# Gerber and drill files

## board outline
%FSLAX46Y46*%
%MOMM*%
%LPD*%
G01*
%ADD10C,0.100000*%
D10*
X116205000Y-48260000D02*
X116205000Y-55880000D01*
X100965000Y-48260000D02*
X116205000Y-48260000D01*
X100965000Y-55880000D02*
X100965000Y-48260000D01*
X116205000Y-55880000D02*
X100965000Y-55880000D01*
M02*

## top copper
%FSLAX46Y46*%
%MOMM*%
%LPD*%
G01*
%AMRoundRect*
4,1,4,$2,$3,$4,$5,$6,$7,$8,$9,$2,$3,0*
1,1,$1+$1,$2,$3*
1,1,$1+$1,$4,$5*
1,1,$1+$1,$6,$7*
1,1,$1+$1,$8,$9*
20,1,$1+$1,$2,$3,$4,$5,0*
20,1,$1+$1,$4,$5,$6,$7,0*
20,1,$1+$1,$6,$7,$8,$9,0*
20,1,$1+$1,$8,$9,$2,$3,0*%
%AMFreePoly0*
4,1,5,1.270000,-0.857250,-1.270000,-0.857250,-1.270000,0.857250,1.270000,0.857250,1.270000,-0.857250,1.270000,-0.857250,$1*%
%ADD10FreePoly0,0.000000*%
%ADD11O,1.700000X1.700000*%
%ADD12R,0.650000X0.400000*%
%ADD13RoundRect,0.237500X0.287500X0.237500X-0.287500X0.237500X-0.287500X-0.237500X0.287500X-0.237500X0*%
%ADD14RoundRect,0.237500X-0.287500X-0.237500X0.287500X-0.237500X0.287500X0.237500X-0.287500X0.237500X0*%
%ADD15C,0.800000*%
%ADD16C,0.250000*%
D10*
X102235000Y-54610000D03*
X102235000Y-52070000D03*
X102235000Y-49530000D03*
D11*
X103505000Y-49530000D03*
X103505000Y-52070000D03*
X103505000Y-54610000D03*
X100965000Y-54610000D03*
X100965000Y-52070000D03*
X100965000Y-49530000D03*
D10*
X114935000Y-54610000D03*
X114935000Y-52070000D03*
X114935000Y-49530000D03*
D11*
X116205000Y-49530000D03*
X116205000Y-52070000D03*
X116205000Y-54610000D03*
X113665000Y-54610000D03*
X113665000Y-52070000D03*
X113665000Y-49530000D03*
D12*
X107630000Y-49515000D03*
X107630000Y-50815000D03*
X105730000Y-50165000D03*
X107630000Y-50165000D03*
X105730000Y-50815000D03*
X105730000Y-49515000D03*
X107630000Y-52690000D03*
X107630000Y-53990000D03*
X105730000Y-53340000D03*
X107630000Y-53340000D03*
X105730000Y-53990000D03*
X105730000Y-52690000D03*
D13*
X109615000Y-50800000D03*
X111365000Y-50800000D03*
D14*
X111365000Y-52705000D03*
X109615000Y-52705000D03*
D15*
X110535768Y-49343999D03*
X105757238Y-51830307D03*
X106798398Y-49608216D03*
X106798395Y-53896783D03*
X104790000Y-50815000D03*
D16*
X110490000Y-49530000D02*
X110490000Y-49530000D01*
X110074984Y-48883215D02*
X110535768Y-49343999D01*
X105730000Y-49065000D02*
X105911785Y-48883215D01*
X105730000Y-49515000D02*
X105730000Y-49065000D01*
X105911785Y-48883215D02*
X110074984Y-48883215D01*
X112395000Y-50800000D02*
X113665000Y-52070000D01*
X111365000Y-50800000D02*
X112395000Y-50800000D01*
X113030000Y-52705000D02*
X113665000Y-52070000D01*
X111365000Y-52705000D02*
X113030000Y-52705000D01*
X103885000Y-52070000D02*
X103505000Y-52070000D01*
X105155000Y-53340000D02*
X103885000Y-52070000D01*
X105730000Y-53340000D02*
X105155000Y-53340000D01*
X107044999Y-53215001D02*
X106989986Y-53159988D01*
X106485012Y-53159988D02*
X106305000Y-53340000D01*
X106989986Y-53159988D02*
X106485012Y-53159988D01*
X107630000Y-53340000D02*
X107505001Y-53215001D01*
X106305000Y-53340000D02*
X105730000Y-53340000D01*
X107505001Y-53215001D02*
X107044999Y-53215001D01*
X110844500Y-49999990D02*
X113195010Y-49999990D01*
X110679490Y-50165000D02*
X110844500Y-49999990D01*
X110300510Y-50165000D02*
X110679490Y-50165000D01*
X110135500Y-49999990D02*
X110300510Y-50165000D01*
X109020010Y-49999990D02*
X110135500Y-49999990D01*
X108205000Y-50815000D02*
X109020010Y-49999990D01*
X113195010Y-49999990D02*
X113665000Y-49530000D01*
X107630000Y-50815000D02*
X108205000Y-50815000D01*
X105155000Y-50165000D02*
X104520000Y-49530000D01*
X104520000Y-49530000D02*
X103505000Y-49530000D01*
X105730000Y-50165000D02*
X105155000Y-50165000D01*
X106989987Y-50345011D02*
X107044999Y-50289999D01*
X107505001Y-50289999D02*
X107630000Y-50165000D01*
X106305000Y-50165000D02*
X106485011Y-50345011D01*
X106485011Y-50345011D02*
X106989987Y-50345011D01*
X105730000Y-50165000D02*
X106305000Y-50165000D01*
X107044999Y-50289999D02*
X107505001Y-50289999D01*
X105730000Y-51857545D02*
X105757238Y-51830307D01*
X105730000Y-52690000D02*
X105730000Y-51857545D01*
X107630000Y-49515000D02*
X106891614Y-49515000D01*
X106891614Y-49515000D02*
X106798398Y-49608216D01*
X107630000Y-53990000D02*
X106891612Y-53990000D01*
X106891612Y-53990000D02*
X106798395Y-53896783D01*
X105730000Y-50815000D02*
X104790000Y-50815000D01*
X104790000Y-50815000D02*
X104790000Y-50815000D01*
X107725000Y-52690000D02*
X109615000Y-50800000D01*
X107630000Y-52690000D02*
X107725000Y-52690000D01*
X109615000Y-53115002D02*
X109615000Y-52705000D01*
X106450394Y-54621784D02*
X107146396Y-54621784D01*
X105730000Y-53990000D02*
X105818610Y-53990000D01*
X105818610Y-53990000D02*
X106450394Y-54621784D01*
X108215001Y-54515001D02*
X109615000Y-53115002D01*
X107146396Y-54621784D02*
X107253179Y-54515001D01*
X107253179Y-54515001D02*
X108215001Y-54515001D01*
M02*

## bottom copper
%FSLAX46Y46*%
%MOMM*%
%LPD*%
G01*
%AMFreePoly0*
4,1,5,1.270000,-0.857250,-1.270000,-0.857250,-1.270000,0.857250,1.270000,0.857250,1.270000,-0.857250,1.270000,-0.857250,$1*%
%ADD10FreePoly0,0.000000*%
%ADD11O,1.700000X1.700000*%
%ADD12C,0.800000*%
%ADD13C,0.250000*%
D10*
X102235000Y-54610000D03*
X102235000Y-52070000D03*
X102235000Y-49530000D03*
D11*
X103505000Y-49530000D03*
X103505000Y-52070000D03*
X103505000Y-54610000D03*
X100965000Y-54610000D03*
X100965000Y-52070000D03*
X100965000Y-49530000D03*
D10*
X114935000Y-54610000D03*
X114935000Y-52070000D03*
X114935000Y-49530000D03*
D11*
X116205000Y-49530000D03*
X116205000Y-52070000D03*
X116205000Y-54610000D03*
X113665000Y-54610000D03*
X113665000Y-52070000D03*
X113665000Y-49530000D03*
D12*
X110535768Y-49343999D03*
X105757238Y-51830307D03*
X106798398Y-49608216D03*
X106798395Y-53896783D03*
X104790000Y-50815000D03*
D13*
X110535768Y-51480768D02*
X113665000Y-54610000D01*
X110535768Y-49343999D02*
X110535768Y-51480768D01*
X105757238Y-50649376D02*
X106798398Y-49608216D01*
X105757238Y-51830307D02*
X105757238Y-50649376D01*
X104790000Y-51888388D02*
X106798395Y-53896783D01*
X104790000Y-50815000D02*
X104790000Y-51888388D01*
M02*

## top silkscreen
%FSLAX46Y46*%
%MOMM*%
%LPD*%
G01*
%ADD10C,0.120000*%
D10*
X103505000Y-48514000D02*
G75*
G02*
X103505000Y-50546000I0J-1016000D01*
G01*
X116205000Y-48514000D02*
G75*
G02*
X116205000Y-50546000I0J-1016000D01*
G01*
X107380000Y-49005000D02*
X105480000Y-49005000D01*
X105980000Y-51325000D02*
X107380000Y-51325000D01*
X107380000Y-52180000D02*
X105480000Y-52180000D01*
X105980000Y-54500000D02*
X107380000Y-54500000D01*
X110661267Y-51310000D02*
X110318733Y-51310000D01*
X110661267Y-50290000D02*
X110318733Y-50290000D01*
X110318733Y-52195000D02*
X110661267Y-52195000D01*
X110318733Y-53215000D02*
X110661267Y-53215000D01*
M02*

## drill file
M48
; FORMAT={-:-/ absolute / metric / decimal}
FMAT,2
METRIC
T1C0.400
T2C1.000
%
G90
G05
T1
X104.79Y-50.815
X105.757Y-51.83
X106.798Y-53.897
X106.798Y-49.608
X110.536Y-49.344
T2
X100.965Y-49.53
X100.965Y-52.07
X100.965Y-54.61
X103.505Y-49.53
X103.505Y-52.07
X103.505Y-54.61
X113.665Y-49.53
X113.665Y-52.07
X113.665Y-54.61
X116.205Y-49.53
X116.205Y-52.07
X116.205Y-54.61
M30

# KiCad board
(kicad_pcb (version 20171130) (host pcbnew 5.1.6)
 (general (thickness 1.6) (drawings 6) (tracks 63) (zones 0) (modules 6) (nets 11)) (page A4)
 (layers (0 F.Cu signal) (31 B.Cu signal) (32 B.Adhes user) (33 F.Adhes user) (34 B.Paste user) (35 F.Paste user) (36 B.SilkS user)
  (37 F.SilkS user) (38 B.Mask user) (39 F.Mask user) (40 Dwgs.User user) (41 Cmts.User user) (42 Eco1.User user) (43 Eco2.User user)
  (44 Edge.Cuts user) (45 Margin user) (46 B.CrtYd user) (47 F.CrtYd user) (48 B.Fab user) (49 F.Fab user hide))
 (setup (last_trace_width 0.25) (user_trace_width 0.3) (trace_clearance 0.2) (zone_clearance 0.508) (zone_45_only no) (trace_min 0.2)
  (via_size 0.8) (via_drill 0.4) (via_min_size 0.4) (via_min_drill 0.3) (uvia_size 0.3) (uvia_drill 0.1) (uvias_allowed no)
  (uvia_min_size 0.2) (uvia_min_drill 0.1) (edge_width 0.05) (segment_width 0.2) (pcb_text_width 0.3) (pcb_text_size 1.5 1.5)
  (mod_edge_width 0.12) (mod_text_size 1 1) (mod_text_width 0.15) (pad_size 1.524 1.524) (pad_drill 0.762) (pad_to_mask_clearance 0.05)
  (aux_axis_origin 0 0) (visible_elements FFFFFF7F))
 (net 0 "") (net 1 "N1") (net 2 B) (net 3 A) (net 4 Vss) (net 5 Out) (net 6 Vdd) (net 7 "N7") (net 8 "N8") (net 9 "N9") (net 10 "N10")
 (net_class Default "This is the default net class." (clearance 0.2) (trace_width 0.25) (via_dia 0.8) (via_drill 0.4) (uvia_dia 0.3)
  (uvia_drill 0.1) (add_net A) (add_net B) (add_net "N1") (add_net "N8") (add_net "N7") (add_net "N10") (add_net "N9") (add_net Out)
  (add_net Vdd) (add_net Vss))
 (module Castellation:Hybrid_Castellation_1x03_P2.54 (layer F.Cu) (at 102.235 49.53)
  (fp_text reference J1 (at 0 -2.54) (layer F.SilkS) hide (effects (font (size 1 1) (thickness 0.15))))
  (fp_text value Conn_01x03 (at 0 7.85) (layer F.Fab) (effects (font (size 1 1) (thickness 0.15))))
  (fp_arc (start 1.27 0) (end 1.27 1.016) (angle -180) (layer F.SilkS) (width 0.12))
  (pad 3 connect custom (at 0 5.08) (size 2.54 1.7145) (layers B.Cu B.Mask) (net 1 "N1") (zone_connect 0)
   (options (clearance outline) (anchor rect)) (primitives))
  (pad 2 connect custom (at 0 2.54) (size 2.54 1.7145) (layers B.Cu B.Mask) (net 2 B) (zone_connect 0)
   (options (clearance outline) (anchor rect)) (primitives))
  (pad 1 connect custom (at 0 0) (size 2.54 1.7145) (layers B.Cu B.Mask) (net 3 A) (zone_connect 0)
   (options (clearance outline) (anchor rect)) (primitives))
  (pad 3 connect custom (at 0 5.08) (size 2.54 1.7145) (layers F.Cu F.Mask) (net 1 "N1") (zone_connect 0)
   (options (clearance outline) (anchor rect)) (primitives))
  (pad 2 connect custom (at 0 2.54) (size 2.54 1.7145) (layers F.Cu F.Mask) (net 2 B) (zone_connect 0)
   (options (clearance outline) (anchor rect)) (primitives))
  (pad 1 connect custom (at 0 0) (size 2.54 1.7145) (layers F.Cu F.Mask) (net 3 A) (zone_connect 0)
   (options (clearance outline) (anchor rect)) (primitives))
  (pad 1 thru_hole oval (at 1.27 0) (size 1.7 1.7) (drill 1) (layers *.Cu *.Mask) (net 3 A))
  (pad 2 thru_hole oval (at 1.27 2.54) (size 1.7 1.7) (drill 1) (layers *.Cu *.Mask) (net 2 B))
  (pad 3 thru_hole oval (at 1.27 5.08) (size 1.7 1.7) (drill 1) (layers *.Cu *.Mask) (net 1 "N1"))
  (pad 3 thru_hole oval (at -1.27 5.08) (size 1.7 1.7) (drill 1) (layers *.Cu *.Mask) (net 1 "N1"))
  (pad 2 thru_hole oval (at -1.27 2.54) (size 1.7 1.7) (drill 1) (layers *.Cu *.Mask) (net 2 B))
  (pad 1 thru_hole oval (at -1.27 0) (size 1.7 1.7) (drill 1) (layers *.Cu *.Mask) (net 3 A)))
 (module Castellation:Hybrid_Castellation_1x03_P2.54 (layer F.Cu) (at 114.935 49.53)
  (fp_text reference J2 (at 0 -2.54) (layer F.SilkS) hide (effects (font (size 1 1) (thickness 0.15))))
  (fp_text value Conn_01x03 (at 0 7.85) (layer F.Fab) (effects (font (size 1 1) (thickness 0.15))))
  (fp_arc (start 1.27 0) (end 1.27 1.016) (angle -180) (layer F.SilkS) (width 0.12))
  (pad 3 connect custom (at 0 5.08) (size 2.54 1.7145) (layers B.Cu B.Mask) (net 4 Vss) (zone_connect 0)
   (options (clearance outline) (anchor rect)) (primitives))
  (pad 2 connect custom (at 0 2.54) (size 2.54 1.7145) (layers B.Cu B.Mask) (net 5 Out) (zone_connect 0)
   (options (clearance outline) (anchor rect)) (primitives))
  (pad 1 connect custom (at 0 0) (size 2.54 1.7145) (layers B.Cu B.Mask) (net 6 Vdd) (zone_connect 0)
   (options (clearance outline) (anchor rect)) (primitives))
  (pad 3 connect custom (at 0 5.08) (size 2.54 1.7145) (layers F.Cu F.Mask) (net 4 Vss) (zone_connect 0)
   (options (clearance outline) (anchor rect)) (primitives))
  (pad 2 connect custom (at 0 2.54) (size 2.54 1.7145) (layers F.Cu F.Mask) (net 5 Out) (zone_connect 0)
   (options (clearance outline) (anchor rect)) (primitives))
  (pad 1 connect custom (at 0 0) (size 2.54 1.7145) (layers F.Cu F.Mask) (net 6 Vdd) (zone_connect 0)
   (options (clearance outline) (anchor rect)) (primitives))
  (pad 1 thru_hole oval (at 1.27 0) (size 1.7 1.7) (drill 1) (layers *.Cu *.Mask) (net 6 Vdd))
  (pad 2 thru_hole oval (at 1.27 2.54) (size 1.7 1.7) (drill 1) (layers *.Cu *.Mask) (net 5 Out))
  (pad 3 thru_hole oval (at 1.27 5.08) (size 1.7 1.7) (drill 1) (layers *.Cu *.Mask) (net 4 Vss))
  (pad 3 thru_hole oval (at -1.27 5.08) (size 1.7 1.7) (drill 1) (layers *.Cu *.Mask) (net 4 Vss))
  (pad 2 thru_hole oval (at -1.27 2.54) (size 1.7 1.7) (drill 1) (layers *.Cu *.Mask) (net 5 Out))
  (pad 1 thru_hole oval (at -1.27 0) (size 1.7 1.7) (drill 1) (layers *.Cu *.Mask) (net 6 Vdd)))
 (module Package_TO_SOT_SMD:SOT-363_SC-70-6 (layer F.Cu) (at 106.68 50.165)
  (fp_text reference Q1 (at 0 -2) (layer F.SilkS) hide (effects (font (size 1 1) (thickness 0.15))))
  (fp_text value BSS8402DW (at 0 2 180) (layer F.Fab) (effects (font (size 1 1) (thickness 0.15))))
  (fp_line (start 0.7 -1.16) (end -1.2 -1.16) (layer F.SilkS) (width 0.12))
  (fp_line (start -0.7 1.16) (end 0.7 1.16) (layer F.SilkS) (width 0.12))
  (pad 6 smd rect (at 0.95 -0.65) (size 0.65 0.4) (layers F.Cu F.Paste F.Mask) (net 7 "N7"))
  (pad 4 smd rect (at 0.95 0.65) (size 0.65 0.4) (layers F.Cu F.Paste F.Mask) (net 6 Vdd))
  (pad 2 smd rect (at -0.95 0) (size 0.65 0.4) (layers F.Cu F.Paste F.Mask) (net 3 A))
  (pad 5 smd rect (at 0.95 0) (size 0.65 0.4) (layers F.Cu F.Paste F.Mask) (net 3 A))
  (pad 3 smd rect (at -0.95 0.65) (size 0.65 0.4) (layers F.Cu F.Paste F.Mask) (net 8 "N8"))
  (pad 1 smd rect (at -0.95 -0.65) (size 0.65 0.4) (layers F.Cu F.Paste F.Mask) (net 4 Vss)))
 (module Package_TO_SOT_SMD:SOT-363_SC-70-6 (layer F.Cu) (at 106.68 53.34)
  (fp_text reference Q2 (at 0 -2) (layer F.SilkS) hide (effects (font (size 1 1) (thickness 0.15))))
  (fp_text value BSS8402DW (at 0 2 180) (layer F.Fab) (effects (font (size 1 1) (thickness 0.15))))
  (fp_line (start 0.7 -1.16) (end -1.2 -1.16) (layer F.SilkS) (width 0.12))
  (fp_line (start -0.7 1.16) (end 0.7 1.16) (layer F.SilkS) (width 0.12))
  (pad 6 smd rect (at 0.95 -0.65) (size 0.65 0.4) (layers F.Cu F.Paste F.Mask) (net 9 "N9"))
  (pad 4 smd rect (at 0.95 0.65) (size 0.65 0.4) (layers F.Cu F.Paste F.Mask) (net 8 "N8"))
  (pad 2 smd rect (at -0.95 0) (size 0.65 0.4) (layers F.Cu F.Paste F.Mask) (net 2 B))
  (pad 5 smd rect (at 0.95 0) (size 0.65 0.4) (layers F.Cu F.Paste F.Mask) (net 2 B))
  (pad 3 smd rect (at -0.95 0.65) (size 0.65 0.4) (layers F.Cu F.Paste F.Mask) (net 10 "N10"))
  (pad 1 smd rect (at -0.95 -0.65) (size 0.65 0.4) (layers F.Cu F.Paste F.Mask) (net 7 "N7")))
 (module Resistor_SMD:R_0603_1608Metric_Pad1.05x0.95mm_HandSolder (layer F.Cu) (at 110.49 50.8 180)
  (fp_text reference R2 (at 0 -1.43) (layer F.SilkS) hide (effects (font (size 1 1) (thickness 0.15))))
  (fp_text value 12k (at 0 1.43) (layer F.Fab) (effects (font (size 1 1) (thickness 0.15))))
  (fp_line (start -0.171267 -0.51) (end 0.171267 -0.51) (layer F.SilkS) (width 0.12))
  (fp_line (start -0.171267 0.51) (end 0.171267 0.51) (layer F.SilkS) (width 0.12))
  (pad 2 smd roundrect (at 0.875 0 180) (size 1.05 0.95) (layers F.Cu F.Paste F.Mask) (roundrect_rratio 0.25) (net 9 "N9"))
  (pad 1 smd roundrect (at -0.875 0 180) (size 1.05 0.95) (layers F.Cu F.Paste F.Mask) (roundrect_rratio 0.25) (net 5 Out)))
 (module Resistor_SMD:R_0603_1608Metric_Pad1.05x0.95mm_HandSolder (layer F.Cu) (at 110.49 52.705)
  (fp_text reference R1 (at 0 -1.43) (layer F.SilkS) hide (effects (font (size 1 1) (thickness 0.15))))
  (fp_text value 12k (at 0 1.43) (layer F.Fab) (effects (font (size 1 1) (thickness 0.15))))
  (fp_line (start -0.171267 -0.51) (end 0.171267 -0.51) (layer F.SilkS) (width 0.12))
  (fp_line (start -0.171267 0.51) (end 0.171267 0.51) (layer F.SilkS) (width 0.12))
  (pad 2 smd roundrect (at 0.875 0) (size 1.05 0.95) (layers F.Cu F.Paste F.Mask) (roundrect_rratio 0.25) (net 5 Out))
  (pad 1 smd roundrect (at -0.875 0) (size 1.05 0.95) (layers F.Cu F.Paste F.Mask) (roundrect_rratio 0.25) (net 10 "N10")))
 (gr_line (start 116.205 48.26) (end 116.205 55.88) (layer Edge.Cuts) (width 0.1))
 (gr_line (start 100.965 48.26) (end 116.205 48.26) (layer Edge.Cuts) (width 0.1))
 (gr_line (start 100.965 55.88) (end 100.965 48.26) (layer Edge.Cuts) (width 0.1))
 (gr_line (start 116.205 55.88) (end 100.965 55.88) (layer Edge.Cuts) (width 0.1))
 (segment (start 110.49 49.53) (end 110.49 49.53) (width 0.25) (layer F.Cu) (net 4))
 (via (at 110.535768 49.343999) (size 0.8) (drill 0.4) (layers F.Cu B.Cu) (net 4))
 (segment (start 110.074984 48.883215) (end 110.535768 49.343999) (width 0.25) (layer F.Cu) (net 4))
 (segment (start 105.73 49.065) (end 105.911785 48.883215) (width 0.25) (layer F.Cu) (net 4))
 (segment (start 105.73 49.515) (end 105.73 49.065) (width 0.25) (layer F.Cu) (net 4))
 (segment (start 105.911785 48.883215) (end 110.074984 48.883215) (width 0.25) (layer F.Cu) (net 4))
 (segment (start 110.535768 51.480768) (end 113.665 54.61) (width 0.25) (layer B.Cu) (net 4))
 (segment (start 110.535768 49.343999) (end 110.535768 51.480768) (width 0.25) (layer B.Cu) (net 4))
 (segment (start 112.395 50.8) (end 113.665 52.07) (width 0.25) (layer F.Cu) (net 5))
 (segment (start 111.365 50.8) (end 112.395 50.8) (width 0.25) (layer F.Cu) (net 5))
 (segment (start 113.03 52.705) (end 113.665 52.07) (width 0.25) (layer F.Cu) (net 5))
 (segment (start 111.365 52.705) (end 113.03 52.705) (width 0.25) (layer F.Cu) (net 5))
 (segment (start 103.885 52.07) (end 103.505 52.07) (width 0.25) (layer F.Cu) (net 2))
 (segment (start 105.155 53.34) (end 103.885 52.07) (width 0.25) (layer F.Cu) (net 2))
 (segment (start 105.73 53.34) (end 105.155 53.34) (width 0.25) (layer F.Cu) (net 2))
 (segment (start 107.044999 53.215001) (end 106.989986 53.159988) (width 0.25) (layer F.Cu) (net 2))
 (segment (start 106.485012 53.159988) (end 106.305 53.34) (width 0.25) (layer F.Cu) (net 2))
 (segment (start 106.989986 53.159988) (end 106.485012 53.159988) (width 0.25) (layer F.Cu) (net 2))
 (segment (start 107.63 53.34) (end 107.505001 53.215001) (width 0.25) (layer F.Cu) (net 2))
 (segment (start 106.305 53.34) (end 105.73 53.34) (width 0.25) (layer F.Cu) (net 2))
 (segment (start 107.505001 53.215001) (end 107.044999 53.215001) (width 0.25) (layer F.Cu) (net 2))
 (segment (start 110.8445 49.99999) (end 113.19501 49.99999) (width 0.25) (layer F.Cu) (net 6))
 (segment (start 110.67949 50.165) (end 110.8445 49.99999) (width 0.25) (layer F.Cu) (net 6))
 (segment (start 110.30051 50.165) (end 110.67949 50.165) (width 0.25) (layer F.Cu) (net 6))
 (segment (start 110.1355 49.99999) (end 110.30051 50.165) (width 0.25) (layer F.Cu) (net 6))
 (segment (start 109.02001 49.99999) (end 110.1355 49.99999) (width 0.25) (layer F.Cu) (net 6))
 (segment (start 108.205 50.815) (end 109.02001 49.99999) (width 0.25) (layer F.Cu) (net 6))
 (segment (start 113.19501 49.99999) (end 113.665 49.53) (width 0.25) (layer F.Cu) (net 6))
 (segment (start 107.63 50.815) (end 108.205 50.815) (width 0.25) (layer F.Cu) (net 6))
 (segment (start 105.155 50.165) (end 104.52 49.53) (width 0.25) (layer F.Cu) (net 3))
 (segment (start 104.52 49.53) (end 103.505 49.53) (width 0.25) (layer F.Cu) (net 3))
 (segment (start 105.73 50.165) (end 105.155 50.165) (width 0.25) (layer F.Cu) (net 3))
 (segment (start 106.989987 50.345011) (end 107.044999 50.289999) (width 0.25) (layer F.Cu) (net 3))
 (segment (start 107.505001 50.289999) (end 107.63 50.165) (width 0.25) (layer F.Cu) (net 3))
 (segment (start 106.305 50.165) (end 106.485011 50.345011) (width 0.25) (layer F.Cu) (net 3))
 (segment (start 106.485011 50.345011) (end 106.989987 50.345011) (width 0.25) (layer F.Cu) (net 3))
 (segment (start 105.73 50.165) (end 106.305 50.165) (width 0.25) (layer F.Cu) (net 3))
 (segment (start 107.044999 50.289999) (end 107.505001 50.289999) (width 0.25) (layer F.Cu) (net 3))
 (via (at 105.757238 51.830307) (size 0.8) (drill 0.4) (layers F.Cu B.Cu) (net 7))
 (segment (start 105.73 51.857545) (end 105.757238 51.830307) (width 0.25) (layer F.Cu) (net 7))
 (segment (start 105.73 52.69) (end 105.73 51.857545) (width 0.25) (layer F.Cu) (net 7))
 (segment (start 107.63 49.515) (end 106.891614 49.515) (width 0.25) (layer F.Cu) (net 7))
 (segment (start 105.757238 50.649376) (end 106.798398 49.608216) (width 0.25) (layer B.Cu) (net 7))
 (segment (start 105.757238 51.830307) (end 105.757238 50.649376) (width 0.25) (layer B.Cu) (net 7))
 (via (at 106.798398 49.608216) (size 0.8) (drill 0.4) (layers F.Cu B.Cu) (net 7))
 (segment (start 106.891614 49.515) (end 106.798398 49.608216) (width 0.25) (layer F.Cu) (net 7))
 (segment (start 107.63 53.99) (end 106.891612 53.99) (width 0.25) (layer F.Cu) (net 8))
 (via (at 106.798395 53.896783) (size 0.8) (drill 0.4) (layers F.Cu B.Cu) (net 8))
 (segment (start 106.891612 53.99) (end 106.798395 53.896783) (width 0.25) (layer F.Cu) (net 8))
 (segment (start 105.73 50.815) (end 104.79 50.815) (width 0.25) (layer F.Cu) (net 8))
 (segment (start 104.79 50.815) (end 104.79 50.815) (width 0.25) (layer F.Cu) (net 8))
 (via (at 104.79 50.815) (size 0.8) (drill 0.4) (layers F.Cu B.Cu) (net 8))
 (segment (start 104.79 51.888388) (end 106.798395 53.896783) (width 0.25) (layer B.Cu) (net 8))
 (segment (start 104.79 50.815) (end 104.79 51.888388) (width 0.25) (layer B.Cu) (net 8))
 (segment (start 107.725 52.69) (end 109.615 50.8) (width 0.25) (layer F.Cu) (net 9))
 (segment (start 107.63 52.69) (end 107.725 52.69) (width 0.25) (layer F.Cu) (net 9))
 (segment (start 109.615 53.115002) (end 109.615 52.705) (width 0.25) (layer F.Cu) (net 10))
 (segment (start 106.450394 54.621784) (end 107.146396 54.621784) (width 0.25) (layer F.Cu) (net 10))
 (segment (start 105.73 53.99) (end 105.81861 53.99) (width 0.25) (layer F.Cu) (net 10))
 (segment (start 105.81861 53.99) (end 106.450394 54.621784) (width 0.25) (layer F.Cu) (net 10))
 (segment (start 108.215001 54.515001) (end 109.615 53.115002) (width 0.25) (layer F.Cu) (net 10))
 (segment (start 107.146396 54.621784) (end 107.253179 54.515001) (width 0.25) (layer F.Cu) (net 10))
 (segment (start 107.253179 54.515001) (end 108.215001 54.515001) (width 0.25) (layer F.Cu) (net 10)))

